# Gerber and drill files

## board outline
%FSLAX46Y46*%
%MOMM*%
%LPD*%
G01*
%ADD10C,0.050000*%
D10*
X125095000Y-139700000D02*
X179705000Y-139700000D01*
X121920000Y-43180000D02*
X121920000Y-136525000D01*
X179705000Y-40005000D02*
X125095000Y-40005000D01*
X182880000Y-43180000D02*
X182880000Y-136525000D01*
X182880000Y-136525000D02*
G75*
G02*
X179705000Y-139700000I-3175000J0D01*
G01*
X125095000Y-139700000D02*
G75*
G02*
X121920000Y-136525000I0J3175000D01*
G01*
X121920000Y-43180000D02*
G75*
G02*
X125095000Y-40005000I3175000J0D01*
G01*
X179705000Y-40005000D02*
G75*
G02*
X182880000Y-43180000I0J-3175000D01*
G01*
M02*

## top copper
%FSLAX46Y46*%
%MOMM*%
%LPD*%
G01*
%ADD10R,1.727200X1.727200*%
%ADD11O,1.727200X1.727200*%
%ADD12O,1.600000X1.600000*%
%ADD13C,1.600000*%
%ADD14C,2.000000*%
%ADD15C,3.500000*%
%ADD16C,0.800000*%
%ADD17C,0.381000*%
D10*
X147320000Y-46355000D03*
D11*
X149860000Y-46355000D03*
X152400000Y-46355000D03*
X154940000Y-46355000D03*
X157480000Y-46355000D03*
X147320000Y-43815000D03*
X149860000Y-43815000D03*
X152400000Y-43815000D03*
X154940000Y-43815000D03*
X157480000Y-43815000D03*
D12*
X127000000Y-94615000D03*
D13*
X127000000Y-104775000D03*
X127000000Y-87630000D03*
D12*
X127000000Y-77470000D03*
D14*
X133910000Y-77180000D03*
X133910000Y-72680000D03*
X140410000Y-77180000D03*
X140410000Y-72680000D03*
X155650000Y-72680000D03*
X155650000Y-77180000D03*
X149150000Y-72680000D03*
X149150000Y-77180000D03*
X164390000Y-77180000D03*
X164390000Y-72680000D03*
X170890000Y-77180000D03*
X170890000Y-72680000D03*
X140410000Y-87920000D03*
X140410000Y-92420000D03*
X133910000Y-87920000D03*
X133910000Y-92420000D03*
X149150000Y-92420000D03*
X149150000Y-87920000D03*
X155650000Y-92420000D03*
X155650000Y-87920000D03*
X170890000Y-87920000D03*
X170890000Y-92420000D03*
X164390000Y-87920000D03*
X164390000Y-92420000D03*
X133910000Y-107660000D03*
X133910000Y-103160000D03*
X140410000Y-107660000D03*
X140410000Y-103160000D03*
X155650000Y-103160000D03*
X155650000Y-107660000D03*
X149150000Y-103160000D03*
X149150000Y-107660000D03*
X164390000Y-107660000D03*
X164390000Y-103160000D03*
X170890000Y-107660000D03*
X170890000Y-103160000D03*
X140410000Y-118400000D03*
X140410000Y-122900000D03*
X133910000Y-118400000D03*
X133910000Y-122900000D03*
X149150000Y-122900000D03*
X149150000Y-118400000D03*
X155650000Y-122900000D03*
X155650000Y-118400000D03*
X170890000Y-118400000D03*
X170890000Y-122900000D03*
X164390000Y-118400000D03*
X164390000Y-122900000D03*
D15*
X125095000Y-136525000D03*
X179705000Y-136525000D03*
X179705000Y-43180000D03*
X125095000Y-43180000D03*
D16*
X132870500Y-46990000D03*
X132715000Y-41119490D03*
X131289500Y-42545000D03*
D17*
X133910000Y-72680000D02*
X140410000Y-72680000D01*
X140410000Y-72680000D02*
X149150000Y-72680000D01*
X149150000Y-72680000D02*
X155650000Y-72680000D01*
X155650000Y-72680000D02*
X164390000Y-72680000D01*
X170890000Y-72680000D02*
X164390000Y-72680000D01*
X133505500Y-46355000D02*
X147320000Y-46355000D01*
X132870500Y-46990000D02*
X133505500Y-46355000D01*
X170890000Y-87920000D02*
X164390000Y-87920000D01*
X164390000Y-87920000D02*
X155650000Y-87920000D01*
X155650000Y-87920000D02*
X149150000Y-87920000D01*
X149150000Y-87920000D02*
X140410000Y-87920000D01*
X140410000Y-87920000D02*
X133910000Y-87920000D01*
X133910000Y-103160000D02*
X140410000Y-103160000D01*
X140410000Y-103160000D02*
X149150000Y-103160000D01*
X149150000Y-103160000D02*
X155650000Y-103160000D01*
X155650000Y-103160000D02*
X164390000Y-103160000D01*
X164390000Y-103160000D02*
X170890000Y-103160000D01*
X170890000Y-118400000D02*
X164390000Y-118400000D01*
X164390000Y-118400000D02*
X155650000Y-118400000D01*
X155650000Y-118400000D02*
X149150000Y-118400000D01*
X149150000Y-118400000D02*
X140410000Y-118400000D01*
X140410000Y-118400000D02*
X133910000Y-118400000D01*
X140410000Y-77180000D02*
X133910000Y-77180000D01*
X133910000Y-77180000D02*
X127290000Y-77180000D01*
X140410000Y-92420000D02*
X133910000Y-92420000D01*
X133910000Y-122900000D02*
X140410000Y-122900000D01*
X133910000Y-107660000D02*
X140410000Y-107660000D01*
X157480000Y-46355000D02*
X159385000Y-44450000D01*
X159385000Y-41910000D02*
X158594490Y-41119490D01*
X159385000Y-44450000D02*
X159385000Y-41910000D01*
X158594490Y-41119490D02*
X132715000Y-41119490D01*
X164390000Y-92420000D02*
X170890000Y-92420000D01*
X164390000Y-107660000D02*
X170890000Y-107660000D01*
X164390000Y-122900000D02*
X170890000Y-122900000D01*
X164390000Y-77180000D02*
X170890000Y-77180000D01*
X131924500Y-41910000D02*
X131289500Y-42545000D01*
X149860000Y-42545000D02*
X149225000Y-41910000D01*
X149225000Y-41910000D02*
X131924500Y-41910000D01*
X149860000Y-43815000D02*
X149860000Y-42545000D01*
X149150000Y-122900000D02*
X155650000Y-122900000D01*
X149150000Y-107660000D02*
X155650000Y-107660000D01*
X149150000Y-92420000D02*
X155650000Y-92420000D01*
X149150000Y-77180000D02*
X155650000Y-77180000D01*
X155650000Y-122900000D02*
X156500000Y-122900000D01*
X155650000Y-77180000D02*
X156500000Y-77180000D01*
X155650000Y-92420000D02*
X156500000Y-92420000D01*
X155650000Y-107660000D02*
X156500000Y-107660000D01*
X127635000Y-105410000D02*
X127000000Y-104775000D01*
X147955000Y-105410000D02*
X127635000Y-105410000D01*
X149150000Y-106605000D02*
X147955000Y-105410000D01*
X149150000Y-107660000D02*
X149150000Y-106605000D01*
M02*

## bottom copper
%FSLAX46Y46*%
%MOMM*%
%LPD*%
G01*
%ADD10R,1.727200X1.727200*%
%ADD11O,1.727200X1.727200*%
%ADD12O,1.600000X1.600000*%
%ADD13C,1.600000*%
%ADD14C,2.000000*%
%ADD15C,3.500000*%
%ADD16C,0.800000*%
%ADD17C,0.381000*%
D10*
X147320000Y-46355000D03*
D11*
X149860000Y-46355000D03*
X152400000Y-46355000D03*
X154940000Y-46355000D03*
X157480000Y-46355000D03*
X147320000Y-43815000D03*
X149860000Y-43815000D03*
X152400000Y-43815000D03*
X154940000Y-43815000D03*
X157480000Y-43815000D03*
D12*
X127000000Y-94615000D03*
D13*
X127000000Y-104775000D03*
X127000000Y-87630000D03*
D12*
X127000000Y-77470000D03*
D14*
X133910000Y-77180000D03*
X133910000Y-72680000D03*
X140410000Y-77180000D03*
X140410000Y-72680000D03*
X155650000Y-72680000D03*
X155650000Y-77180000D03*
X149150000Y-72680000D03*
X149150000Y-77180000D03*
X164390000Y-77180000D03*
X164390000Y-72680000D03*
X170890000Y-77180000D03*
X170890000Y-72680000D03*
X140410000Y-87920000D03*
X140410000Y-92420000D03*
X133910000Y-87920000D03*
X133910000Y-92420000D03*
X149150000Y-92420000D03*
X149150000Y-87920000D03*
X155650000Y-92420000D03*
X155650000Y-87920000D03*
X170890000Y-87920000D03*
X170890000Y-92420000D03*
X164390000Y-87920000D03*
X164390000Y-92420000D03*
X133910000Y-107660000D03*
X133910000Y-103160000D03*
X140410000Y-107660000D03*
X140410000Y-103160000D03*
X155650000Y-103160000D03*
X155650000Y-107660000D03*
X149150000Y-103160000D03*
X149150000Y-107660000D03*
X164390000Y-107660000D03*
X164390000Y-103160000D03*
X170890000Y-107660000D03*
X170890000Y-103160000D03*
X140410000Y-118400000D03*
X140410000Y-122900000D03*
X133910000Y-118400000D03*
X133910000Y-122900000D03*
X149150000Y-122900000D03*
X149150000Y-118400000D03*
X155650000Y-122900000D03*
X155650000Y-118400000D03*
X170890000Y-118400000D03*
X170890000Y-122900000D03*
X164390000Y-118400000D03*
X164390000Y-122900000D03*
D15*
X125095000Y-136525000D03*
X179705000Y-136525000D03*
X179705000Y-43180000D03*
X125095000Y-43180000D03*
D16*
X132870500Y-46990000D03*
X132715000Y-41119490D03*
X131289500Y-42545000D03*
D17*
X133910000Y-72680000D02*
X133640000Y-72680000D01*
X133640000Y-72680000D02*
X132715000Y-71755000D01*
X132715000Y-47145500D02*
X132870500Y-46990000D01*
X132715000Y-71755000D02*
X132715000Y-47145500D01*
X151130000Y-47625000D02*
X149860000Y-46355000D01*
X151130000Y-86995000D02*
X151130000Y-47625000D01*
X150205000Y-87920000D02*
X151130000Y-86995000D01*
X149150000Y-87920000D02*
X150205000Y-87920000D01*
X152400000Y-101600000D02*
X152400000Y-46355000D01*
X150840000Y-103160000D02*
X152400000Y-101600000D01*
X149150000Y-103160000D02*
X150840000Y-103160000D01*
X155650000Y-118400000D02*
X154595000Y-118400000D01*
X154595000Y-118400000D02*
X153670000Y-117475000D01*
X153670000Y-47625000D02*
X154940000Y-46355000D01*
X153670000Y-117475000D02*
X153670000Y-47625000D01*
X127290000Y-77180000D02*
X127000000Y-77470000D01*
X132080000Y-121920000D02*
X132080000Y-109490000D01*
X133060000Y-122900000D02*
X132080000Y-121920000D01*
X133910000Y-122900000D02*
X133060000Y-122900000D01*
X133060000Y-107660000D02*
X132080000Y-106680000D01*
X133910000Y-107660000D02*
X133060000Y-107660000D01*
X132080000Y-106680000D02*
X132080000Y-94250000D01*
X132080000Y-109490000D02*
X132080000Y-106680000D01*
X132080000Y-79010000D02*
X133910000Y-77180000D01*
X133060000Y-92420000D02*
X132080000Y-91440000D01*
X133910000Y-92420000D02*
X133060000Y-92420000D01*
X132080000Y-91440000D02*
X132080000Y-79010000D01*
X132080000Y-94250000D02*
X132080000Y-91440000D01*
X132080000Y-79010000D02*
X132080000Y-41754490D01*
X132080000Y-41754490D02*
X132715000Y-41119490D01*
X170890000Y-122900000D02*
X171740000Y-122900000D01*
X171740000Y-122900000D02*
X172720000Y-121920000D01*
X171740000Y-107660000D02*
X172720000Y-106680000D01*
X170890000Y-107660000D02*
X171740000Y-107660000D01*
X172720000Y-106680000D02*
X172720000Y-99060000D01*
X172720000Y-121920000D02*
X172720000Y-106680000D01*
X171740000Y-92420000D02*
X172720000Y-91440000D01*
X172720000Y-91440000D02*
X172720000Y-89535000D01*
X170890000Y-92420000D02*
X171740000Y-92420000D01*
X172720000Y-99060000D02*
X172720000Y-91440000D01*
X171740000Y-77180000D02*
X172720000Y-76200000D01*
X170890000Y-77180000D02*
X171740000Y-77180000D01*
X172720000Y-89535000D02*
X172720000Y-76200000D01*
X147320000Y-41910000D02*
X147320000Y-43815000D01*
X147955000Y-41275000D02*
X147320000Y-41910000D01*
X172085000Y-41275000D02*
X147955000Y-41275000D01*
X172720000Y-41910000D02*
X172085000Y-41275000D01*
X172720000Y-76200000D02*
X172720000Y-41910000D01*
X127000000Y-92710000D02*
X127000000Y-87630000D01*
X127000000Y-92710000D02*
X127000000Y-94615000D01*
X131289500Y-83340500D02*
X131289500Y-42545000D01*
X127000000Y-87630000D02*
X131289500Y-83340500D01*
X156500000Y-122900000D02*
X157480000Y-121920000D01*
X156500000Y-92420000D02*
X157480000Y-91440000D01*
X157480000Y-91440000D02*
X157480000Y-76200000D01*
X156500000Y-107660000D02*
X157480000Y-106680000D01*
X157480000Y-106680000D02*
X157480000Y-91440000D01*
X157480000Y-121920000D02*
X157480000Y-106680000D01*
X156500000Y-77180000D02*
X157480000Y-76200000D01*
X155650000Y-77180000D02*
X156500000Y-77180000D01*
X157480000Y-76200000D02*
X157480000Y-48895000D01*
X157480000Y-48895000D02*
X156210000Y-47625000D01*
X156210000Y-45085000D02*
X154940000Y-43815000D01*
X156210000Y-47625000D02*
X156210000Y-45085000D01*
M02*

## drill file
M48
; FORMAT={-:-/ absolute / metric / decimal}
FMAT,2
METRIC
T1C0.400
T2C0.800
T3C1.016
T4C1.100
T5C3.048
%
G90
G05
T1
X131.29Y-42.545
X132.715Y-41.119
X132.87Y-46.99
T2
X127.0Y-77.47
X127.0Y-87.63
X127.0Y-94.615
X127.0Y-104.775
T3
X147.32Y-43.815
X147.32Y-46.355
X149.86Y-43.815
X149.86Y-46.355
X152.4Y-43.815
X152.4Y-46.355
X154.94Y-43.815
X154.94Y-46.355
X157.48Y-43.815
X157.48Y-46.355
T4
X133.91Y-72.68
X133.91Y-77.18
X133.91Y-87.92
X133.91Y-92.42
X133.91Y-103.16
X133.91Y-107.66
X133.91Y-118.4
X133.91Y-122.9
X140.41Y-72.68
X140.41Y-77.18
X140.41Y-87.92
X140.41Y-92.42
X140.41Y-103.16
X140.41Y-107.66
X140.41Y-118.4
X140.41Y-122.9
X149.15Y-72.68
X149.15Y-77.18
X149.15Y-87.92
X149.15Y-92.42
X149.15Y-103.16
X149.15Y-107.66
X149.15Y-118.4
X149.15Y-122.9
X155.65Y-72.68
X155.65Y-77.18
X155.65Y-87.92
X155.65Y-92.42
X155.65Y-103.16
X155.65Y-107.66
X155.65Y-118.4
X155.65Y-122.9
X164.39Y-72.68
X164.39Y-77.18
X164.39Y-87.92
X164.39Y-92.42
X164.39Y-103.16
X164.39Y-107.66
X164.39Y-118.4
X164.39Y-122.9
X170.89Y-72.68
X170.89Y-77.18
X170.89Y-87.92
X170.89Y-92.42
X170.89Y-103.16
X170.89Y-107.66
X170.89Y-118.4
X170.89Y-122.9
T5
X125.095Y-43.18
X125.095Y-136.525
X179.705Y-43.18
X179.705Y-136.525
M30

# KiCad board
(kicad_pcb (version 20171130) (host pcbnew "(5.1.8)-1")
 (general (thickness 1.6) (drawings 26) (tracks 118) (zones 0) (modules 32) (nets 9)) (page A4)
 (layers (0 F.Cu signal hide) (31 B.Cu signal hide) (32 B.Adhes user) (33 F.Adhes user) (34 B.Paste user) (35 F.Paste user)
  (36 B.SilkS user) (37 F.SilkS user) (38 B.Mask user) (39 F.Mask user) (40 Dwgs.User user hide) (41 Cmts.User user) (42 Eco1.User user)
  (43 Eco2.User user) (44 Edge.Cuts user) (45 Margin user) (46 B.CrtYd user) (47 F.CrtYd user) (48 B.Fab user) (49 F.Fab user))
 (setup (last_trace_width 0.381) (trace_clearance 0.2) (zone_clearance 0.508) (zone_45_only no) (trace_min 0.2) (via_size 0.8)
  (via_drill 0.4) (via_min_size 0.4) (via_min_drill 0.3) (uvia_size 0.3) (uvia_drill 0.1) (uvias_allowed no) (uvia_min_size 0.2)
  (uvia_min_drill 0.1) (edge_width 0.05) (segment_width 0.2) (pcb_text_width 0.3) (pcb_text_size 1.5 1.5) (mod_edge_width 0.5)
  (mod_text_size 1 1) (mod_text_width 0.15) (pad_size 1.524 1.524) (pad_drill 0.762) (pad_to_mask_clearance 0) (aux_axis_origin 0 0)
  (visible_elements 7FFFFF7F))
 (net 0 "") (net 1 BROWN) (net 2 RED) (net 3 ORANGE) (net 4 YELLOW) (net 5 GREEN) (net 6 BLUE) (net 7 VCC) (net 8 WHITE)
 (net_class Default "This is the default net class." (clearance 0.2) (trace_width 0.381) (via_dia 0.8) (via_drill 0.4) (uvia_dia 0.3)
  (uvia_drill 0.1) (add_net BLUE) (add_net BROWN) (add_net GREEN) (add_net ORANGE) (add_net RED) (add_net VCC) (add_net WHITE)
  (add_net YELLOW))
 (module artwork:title (layer F.Cu) (at 152.4 59.055)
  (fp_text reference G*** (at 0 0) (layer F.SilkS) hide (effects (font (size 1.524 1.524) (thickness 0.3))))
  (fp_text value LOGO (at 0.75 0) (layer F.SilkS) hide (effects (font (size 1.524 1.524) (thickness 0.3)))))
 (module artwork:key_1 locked (layer F.Cu) (at 137.16 69.85)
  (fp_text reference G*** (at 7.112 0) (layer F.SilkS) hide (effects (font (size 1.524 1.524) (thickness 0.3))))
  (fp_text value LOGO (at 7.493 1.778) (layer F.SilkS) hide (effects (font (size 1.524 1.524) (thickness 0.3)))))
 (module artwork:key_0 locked (layer F.Cu) (at 152.4 115.57)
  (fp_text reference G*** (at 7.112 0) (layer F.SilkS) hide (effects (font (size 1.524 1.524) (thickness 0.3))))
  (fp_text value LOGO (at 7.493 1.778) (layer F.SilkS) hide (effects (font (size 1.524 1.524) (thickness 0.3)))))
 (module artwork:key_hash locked (layer F.Cu) (at 167.64 115.57)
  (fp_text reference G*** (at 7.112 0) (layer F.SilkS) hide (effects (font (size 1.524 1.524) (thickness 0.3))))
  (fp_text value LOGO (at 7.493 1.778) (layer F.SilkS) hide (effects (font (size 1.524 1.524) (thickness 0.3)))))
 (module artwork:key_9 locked (layer F.Cu) (at 167.64 100.33)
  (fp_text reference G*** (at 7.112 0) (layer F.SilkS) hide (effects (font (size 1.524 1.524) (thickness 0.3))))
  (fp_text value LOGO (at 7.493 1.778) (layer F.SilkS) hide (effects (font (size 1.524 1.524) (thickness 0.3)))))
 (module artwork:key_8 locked (layer F.Cu) (at 152.4 100.33)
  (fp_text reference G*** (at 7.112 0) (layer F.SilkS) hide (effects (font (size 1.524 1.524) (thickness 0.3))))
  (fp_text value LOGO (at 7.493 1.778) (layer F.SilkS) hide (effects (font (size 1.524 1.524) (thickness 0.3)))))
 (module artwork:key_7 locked (layer F.Cu) (at 137.16 100.33)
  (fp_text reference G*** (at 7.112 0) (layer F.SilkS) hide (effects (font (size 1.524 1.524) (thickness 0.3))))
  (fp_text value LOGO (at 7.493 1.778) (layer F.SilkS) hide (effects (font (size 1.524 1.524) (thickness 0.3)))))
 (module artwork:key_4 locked (layer F.Cu) (at 137.16 85.09)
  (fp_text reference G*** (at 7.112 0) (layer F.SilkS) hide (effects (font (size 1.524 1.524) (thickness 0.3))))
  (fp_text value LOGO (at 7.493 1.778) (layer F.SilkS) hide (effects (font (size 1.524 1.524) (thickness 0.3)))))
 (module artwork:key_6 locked (layer F.Cu) (at 167.64 85.09)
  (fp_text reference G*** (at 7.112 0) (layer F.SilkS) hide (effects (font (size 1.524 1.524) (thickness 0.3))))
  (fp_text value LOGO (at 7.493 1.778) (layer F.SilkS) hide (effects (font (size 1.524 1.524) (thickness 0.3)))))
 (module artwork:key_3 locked (layer F.Cu) (at 167.64 69.85)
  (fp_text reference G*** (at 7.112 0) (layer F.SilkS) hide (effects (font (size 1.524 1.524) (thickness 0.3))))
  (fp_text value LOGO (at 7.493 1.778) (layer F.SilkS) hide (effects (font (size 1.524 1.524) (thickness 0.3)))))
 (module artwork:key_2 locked (layer F.Cu) (at 152.4 69.85)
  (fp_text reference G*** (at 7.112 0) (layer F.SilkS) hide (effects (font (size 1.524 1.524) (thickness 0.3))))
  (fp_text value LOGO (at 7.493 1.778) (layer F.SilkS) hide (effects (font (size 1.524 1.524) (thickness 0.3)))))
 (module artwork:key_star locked (layer F.Cu) (at 137.16 115.57)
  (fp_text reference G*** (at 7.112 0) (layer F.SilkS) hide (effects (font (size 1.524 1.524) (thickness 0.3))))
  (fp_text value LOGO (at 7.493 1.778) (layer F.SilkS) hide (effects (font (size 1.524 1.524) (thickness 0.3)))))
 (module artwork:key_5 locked (layer F.Cu) (at 152.4 85.09)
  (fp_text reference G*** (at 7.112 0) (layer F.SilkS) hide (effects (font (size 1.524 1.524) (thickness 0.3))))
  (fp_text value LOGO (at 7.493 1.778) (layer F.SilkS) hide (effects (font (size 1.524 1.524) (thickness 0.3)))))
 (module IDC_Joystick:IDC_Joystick (layer F.Cu) (at 147.32 46.355 90)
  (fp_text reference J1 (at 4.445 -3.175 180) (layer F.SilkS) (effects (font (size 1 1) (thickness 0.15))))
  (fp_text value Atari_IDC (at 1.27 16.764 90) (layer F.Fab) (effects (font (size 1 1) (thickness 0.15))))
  (pad 1 thru_hole rect (at 0 0 90) (size 1.7272 1.7272) (drill 1.016) (layers *.Cu *.Mask) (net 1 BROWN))
  (pad 2 thru_hole oval (at 0 2.54 90) (size 1.7272 1.7272) (drill 1.016) (layers *.Cu *.Mask) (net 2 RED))
  (pad 3 thru_hole oval (at 0 5.08 90) (size 1.7272 1.7272) (drill 1.016) (layers *.Cu *.Mask) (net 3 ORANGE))
  (pad 4 thru_hole oval (at 0 7.62 90) (size 1.7272 1.7272) (drill 1.016) (layers *.Cu *.Mask) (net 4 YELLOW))
  (pad 5 thru_hole oval (at 0 10.16 90) (size 1.7272 1.7272) (drill 1.016) (layers *.Cu *.Mask) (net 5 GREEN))
  (pad 6 thru_hole oval (at 2.54 0 90) (size 1.7272 1.7272) (drill 1.016) (layers *.Cu *.Mask) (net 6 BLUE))
  (pad 7 thru_hole oval (at 2.54 2.54 90) (size 1.7272 1.7272) (drill 1.016) (layers *.Cu *.Mask) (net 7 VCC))
  (pad 8 thru_hole oval (at 2.54 5.08 90) (size 1.7272 1.7272) (drill 1.016) (layers *.Cu *.Mask))
  (pad 9 thru_hole oval (at 2.54 7.62 90) (size 1.7272 1.7272) (drill 1.016) (layers *.Cu *.Mask) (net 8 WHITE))
  (pad 10 thru_hole oval (at 2.54 10.16 90) (size 1.7272 1.7272) (drill 1.016) (layers *.Cu *.Mask)))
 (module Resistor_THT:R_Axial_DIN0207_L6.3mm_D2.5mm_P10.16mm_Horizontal (layer F.Cu) (at 127 104.775 90)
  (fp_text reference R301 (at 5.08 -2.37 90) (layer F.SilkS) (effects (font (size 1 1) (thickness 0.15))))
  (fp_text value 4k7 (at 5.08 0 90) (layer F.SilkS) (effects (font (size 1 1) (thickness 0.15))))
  (pad 2 thru_hole oval (at 10.16 0 90) (size 1.6 1.6) (drill 0.8) (layers *.Cu *.Mask) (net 7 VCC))
  (pad 1 thru_hole circle (at 0 0 90) (size 1.6 1.6) (drill 0.8) (layers *.Cu *.Mask) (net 8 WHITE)))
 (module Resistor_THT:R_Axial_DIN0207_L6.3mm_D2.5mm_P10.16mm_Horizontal (layer F.Cu) (at 127 87.63 90)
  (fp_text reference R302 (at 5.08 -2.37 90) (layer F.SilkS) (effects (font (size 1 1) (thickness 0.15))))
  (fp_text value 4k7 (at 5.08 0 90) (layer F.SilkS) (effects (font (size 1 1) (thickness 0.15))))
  (pad 1 thru_hole circle (at 0 0 90) (size 1.6 1.6) (drill 0.8) (layers *.Cu *.Mask) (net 7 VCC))
  (pad 2 thru_hole oval (at 10.16 0 90) (size 1.6 1.6) (drill 0.8) (layers *.Cu *.Mask) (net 5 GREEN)))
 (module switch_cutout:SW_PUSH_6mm (layer F.Cu) (at 137.16 74.93)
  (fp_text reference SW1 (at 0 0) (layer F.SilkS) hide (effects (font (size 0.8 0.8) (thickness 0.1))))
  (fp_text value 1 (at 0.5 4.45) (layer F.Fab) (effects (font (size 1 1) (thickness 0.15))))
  (pad 2 thru_hole circle (at -3.25 2.25 90) (size 2 2) (drill 1.1) (layers *.Cu *.Mask) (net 5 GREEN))
  (pad 1 thru_hole circle (at -3.25 -2.25 90) (size 2 2) (drill 1.1) (layers *.Cu *.Mask) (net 1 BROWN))
  (pad 2 thru_hole circle (at 3.25 2.25 90) (size 2 2) (drill 1.1) (layers *.Cu *.Mask) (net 5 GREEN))
  (pad 1 thru_hole circle (at 3.25 -2.25 90) (size 2 2) (drill 1.1) (layers *.Cu *.Mask) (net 1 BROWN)))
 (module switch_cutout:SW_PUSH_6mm (layer F.Cu) (at 152.4 74.93)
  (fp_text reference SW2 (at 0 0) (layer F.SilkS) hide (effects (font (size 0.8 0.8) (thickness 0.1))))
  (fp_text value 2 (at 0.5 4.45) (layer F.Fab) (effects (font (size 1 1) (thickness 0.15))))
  (pad 1 thru_hole circle (at 3.25 -2.25 90) (size 2 2) (drill 1.1) (layers *.Cu *.Mask) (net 1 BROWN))
  (pad 2 thru_hole circle (at 3.25 2.25 90) (size 2 2) (drill 1.1) (layers *.Cu *.Mask) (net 8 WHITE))
  (pad 1 thru_hole circle (at -3.25 -2.25 90) (size 2 2) (drill 1.1) (layers *.Cu *.Mask) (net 1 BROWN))
  (pad 2 thru_hole circle (at -3.25 2.25 90) (size 2 2) (drill 1.1) (layers *.Cu *.Mask) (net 8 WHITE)))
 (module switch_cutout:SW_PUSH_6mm (layer F.Cu) (at 167.64 74.93)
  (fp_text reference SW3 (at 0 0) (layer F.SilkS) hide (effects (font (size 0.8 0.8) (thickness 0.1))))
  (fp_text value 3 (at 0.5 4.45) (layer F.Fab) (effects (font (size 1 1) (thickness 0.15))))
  (pad 2 thru_hole circle (at -3.25 2.25 90) (size 2 2) (drill 1.1) (layers *.Cu *.Mask) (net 6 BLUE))
  (pad 1 thru_hole circle (at -3.25 -2.25 90) (size 2 2) (drill 1.1) (layers *.Cu *.Mask) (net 1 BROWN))
  (pad 2 thru_hole circle (at 3.25 2.25 90) (size 2 2) (drill 1.1) (layers *.Cu *.Mask) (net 6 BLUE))
  (pad 1 thru_hole circle (at 3.25 -2.25 90) (size 2 2) (drill 1.1) (layers *.Cu *.Mask) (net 1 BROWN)))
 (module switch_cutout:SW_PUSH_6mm (layer F.Cu) (at 137.16 90.17)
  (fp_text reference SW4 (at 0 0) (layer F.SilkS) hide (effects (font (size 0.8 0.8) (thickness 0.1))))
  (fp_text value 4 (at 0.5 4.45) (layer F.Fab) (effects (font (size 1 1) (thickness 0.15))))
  (pad 1 thru_hole circle (at 3.25 -2.25 90) (size 2 2) (drill 1.1) (layers *.Cu *.Mask) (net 2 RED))
  (pad 2 thru_hole circle (at 3.25 2.25 90) (size 2 2) (drill 1.1) (layers *.Cu *.Mask) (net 5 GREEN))
  (pad 1 thru_hole circle (at -3.25 -2.25 90) (size 2 2) (drill 1.1) (layers *.Cu *.Mask) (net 2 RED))
  (pad 2 thru_hole circle (at -3.25 2.25 90) (size 2 2) (drill 1.1) (layers *.Cu *.Mask) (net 5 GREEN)))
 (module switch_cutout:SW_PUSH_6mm (layer F.Cu) (at 152.4 90.17)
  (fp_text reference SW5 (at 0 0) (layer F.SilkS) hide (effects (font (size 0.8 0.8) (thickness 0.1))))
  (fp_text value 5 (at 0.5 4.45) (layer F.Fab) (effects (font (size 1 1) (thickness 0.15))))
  (pad 2 thru_hole circle (at -3.25 2.25 90) (size 2 2) (drill 1.1) (layers *.Cu *.Mask) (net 8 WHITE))
  (pad 1 thru_hole circle (at -3.25 -2.25 90) (size 2 2) (drill 1.1) (layers *.Cu *.Mask) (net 2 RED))
  (pad 2 thru_hole circle (at 3.25 2.25 90) (size 2 2) (drill 1.1) (layers *.Cu *.Mask) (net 8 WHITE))
  (pad 1 thru_hole circle (at 3.25 -2.25 90) (size 2 2) (drill 1.1) (layers *.Cu *.Mask) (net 2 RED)))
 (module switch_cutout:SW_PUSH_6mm (layer F.Cu) (at 167.64 90.17)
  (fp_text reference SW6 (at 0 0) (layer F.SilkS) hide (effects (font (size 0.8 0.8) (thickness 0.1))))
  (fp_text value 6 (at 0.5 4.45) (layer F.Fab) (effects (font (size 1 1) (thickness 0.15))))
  (pad 1 thru_hole circle (at 3.25 -2.25 90) (size 2 2) (drill 1.1) (layers *.Cu *.Mask) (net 2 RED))
  (pad 2 thru_hole circle (at 3.25 2.25 90) (size 2 2) (drill 1.1) (layers *.Cu *.Mask) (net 6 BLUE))
  (pad 1 thru_hole circle (at -3.25 -2.25 90) (size 2 2) (drill 1.1) (layers *.Cu *.Mask) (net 2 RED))
  (pad 2 thru_hole circle (at -3.25 2.25 90) (size 2 2) (drill 1.1) (layers *.Cu *.Mask) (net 6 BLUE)))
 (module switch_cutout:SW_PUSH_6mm (layer F.Cu) (at 137.16 105.41)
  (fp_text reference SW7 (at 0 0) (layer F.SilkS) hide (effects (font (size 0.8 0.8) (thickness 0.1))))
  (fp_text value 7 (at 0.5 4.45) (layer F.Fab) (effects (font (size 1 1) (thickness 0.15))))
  (pad 2 thru_hole circle (at -3.25 2.25 90) (size 2 2) (drill 1.1) (layers *.Cu *.Mask) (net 5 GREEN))
  (pad 1 thru_hole circle (at -3.25 -2.25 90) (size 2 2) (drill 1.1) (layers *.Cu *.Mask) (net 3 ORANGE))
  (pad 2 thru_hole circle (at 3.25 2.25 90) (size 2 2) (drill 1.1) (layers *.Cu *.Mask) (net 5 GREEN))
  (pad 1 thru_hole circle (at 3.25 -2.25 90) (size 2 2) (drill 1.1) (layers *.Cu *.Mask) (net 3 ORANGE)))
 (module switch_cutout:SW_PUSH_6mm (layer F.Cu) (at 152.4 105.41)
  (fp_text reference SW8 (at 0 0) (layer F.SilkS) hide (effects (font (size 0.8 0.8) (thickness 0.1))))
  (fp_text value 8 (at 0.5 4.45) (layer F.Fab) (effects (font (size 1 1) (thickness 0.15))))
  (pad 1 thru_hole circle (at 3.25 -2.25 90) (size 2 2) (drill 1.1) (layers *.Cu *.Mask) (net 3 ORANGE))
  (pad 2 thru_hole circle (at 3.25 2.25 90) (size 2 2) (drill 1.1) (layers *.Cu *.Mask) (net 8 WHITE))
  (pad 1 thru_hole circle (at -3.25 -2.25 90) (size 2 2) (drill 1.1) (layers *.Cu *.Mask) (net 3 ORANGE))
  (pad 2 thru_hole circle (at -3.25 2.25 90) (size 2 2) (drill 1.1) (layers *.Cu *.Mask) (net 8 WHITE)))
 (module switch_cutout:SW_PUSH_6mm (layer F.Cu) (at 167.64 105.41)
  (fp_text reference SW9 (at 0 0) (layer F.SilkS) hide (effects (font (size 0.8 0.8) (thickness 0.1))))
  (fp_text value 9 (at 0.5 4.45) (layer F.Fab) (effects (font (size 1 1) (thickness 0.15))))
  (pad 2 thru_hole circle (at -3.25 2.25 90) (size 2 2) (drill 1.1) (layers *.Cu *.Mask) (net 6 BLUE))
  (pad 1 thru_hole circle (at -3.25 -2.25 90) (size 2 2) (drill 1.1) (layers *.Cu *.Mask) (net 3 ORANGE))
  (pad 2 thru_hole circle (at 3.25 2.25 90) (size 2 2) (drill 1.1) (layers *.Cu *.Mask) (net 6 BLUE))
  (pad 1 thru_hole circle (at 3.25 -2.25 90) (size 2 2) (drill 1.1) (layers *.Cu *.Mask) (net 3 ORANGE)))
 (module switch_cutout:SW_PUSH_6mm (layer F.Cu) (at 137.16 120.65)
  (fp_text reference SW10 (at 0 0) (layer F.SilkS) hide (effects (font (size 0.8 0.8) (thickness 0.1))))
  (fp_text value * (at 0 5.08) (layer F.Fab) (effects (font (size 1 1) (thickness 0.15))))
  (pad 1 thru_hole circle (at 3.25 -2.25 90) (size 2 2) (drill 1.1) (layers *.Cu *.Mask) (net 4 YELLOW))
  (pad 2 thru_hole circle (at 3.25 2.25 90) (size 2 2) (drill 1.1) (layers *.Cu *.Mask) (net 5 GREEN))
  (pad 1 thru_hole circle (at -3.25 -2.25 90) (size 2 2) (drill 1.1) (layers *.Cu *.Mask) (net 4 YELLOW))
  (pad 2 thru_hole circle (at -3.25 2.25 90) (size 2 2) (drill 1.1) (layers *.Cu *.Mask) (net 5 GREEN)))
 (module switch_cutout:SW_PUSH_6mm (layer F.Cu) (at 152.4 120.65)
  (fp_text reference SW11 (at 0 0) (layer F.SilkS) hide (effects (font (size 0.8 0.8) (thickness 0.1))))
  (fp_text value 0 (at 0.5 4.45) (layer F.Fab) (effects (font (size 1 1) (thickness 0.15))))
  (pad 2 thru_hole circle (at -3.25 2.25 90) (size 2 2) (drill 1.1) (layers *.Cu *.Mask) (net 8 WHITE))
  (pad 1 thru_hole circle (at -3.25 -2.25 90) (size 2 2) (drill 1.1) (layers *.Cu *.Mask) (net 4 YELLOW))
  (pad 2 thru_hole circle (at 3.25 2.25 90) (size 2 2) (drill 1.1) (layers *.Cu *.Mask) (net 8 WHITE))
  (pad 1 thru_hole circle (at 3.25 -2.25 90) (size 2 2) (drill 1.1) (layers *.Cu *.Mask) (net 4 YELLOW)))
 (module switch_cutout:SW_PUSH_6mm (layer F.Cu) (at 167.64 120.65)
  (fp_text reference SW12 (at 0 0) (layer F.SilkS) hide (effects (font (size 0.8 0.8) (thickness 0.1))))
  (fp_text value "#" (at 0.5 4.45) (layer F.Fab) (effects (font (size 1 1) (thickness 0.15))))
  (pad 1 thru_hole circle (at 3.25 -2.25 90) (size 2 2) (drill 1.1) (layers *.Cu *.Mask) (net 4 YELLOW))
  (pad 2 thru_hole circle (at 3.25 2.25 90) (size 2 2) (drill 1.1) (layers *.Cu *.Mask) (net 6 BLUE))
  (pad 1 thru_hole circle (at -3.25 -2.25 90) (size 2 2) (drill 1.1) (layers *.Cu *.Mask) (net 4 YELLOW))
  (pad 2 thru_hole circle (at -3.25 2.25 90) (size 2 2) (drill 1.1) (layers *.Cu *.Mask) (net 6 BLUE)))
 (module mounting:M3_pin (layer F.Cu) (at 125.095 136.525)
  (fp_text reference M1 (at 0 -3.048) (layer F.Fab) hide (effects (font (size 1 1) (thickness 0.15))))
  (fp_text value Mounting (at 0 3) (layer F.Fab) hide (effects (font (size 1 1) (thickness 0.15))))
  (pad 1 thru_hole circle (at 0 0) (size 3.5 3.5) (drill 3.048) (layers *.Cu *.Mask) (solder_mask_margin 0.8)))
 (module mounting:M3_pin (layer F.Cu) (at 179.705 136.525)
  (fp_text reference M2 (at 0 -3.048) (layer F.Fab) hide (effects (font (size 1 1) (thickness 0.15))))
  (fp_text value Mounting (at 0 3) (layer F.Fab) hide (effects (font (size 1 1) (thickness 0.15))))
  (pad 1 thru_hole circle (at 0 0) (size 3.5 3.5) (drill 3.048) (layers *.Cu *.Mask) (solder_mask_margin 0.8)))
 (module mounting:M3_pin (layer F.Cu) (at 179.705 43.18)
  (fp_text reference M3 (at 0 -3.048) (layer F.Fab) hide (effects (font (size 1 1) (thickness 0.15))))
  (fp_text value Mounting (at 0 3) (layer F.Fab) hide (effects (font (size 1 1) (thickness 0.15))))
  (pad 1 thru_hole circle (at 0 0) (size 3.5 3.5) (drill 3.048) (layers *.Cu *.Mask) (solder_mask_margin 0.8)))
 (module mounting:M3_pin (layer F.Cu) (at 125.095 43.18)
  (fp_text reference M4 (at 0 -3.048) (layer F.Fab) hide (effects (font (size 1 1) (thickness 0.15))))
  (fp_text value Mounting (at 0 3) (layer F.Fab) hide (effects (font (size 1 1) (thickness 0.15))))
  (pad 1 thru_hole circle (at 0 0) (size 3.5 3.5) (drill 3.048) (layers *.Cu *.Mask) (solder_mask_margin 0.8)))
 (gr_line (start 125.095 139.7) (end 179.705 139.7) (layer Edge.Cuts) (width 0.05))
 (gr_line (start 121.92 43.18) (end 121.92 136.525) (layer Edge.Cuts) (width 0.05))
 (gr_line (start 179.705 40.005) (end 125.095 40.005) (layer Edge.Cuts) (width 0.05))
 (gr_line (start 182.88 43.18) (end 182.88 136.525) (layer Edge.Cuts) (width 0.05))
 (gr_arc (start 179.705 136.525) (end 179.705 139.7) (angle -90) (layer Edge.Cuts) (width 0.05))
 (gr_arc (start 125.095 136.525) (end 121.92 136.525) (angle -90) (layer Edge.Cuts) (width 0.05))
 (gr_arc (start 125.095 43.18) (end 125.095 40.005) (angle -90) (layer Edge.Cuts) (width 0.05))
 (gr_arc (start 179.705 43.18) (end 182.88 43.18) (angle -90) (layer Edge.Cuts) (width 0.05))
 (segment (start 133.91 72.68) (end 140.41 72.68) (width 0.381) (layer F.Cu) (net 1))
 (segment (start 140.41 72.68) (end 149.15 72.68) (width 0.381) (layer F.Cu) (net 1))
 (segment (start 149.15 72.68) (end 155.65 72.68) (width 0.381) (layer F.Cu) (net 1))
 (segment (start 155.65 72.68) (end 164.39 72.68) (width 0.381) (layer F.Cu) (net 1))
 (segment (start 170.89 72.68) (end 164.39 72.68) (width 0.381) (layer F.Cu) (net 1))
 (segment (start 133.91 72.68) (end 133.64 72.68) (width 0.381) (layer B.Cu) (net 1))
 (segment (start 133.64 72.68) (end 132.715 71.755) (width 0.381) (layer B.Cu) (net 1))
 (via (at 132.8705 46.99) (size 0.8) (drill 0.4) (layers F.Cu B.Cu) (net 1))
 (segment (start 132.715 47.1455) (end 132.8705 46.99) (width 0.381) (layer B.Cu) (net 1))
 (segment (start 132.715 71.755) (end 132.715 47.1455) (width 0.381) (layer B.Cu) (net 1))
 (segment (start 133.5055 46.355) (end 147.32 46.355) (width 0.381) (layer F.Cu) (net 1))
 (segment (start 132.8705 46.99) (end 133.5055 46.355) (width 0.381) (layer F.Cu) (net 1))
 (segment (start 170.89 87.92) (end 164.39 87.92) (width 0.381) (layer F.Cu) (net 2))
 (segment (start 164.39 87.92) (end 155.65 87.92) (width 0.381) (layer F.Cu) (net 2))
 (segment (start 155.65 87.92) (end 149.15 87.92) (width 0.381) (layer F.Cu) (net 2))
 (segment (start 149.15 87.92) (end 140.41 87.92) (width 0.381) (layer F.Cu) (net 2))
 (segment (start 140.41 87.92) (end 133.91 87.92) (width 0.381) (layer F.Cu) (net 2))
 (segment (start 151.13 47.625) (end 149.86 46.355) (width 0.381) (layer B.Cu) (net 2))
 (segment (start 151.13 86.995) (end 151.13 47.625) (width 0.381) (layer B.Cu) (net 2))
 (segment (start 150.205 87.92) (end 151.13 86.995) (width 0.381) (layer B.Cu) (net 2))
 (segment (start 149.15 87.92) (end 150.205 87.92) (width 0.381) (layer B.Cu) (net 2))
 (segment (start 133.91 103.16) (end 140.41 103.16) (width 0.381) (layer F.Cu) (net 3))
 (segment (start 140.41 103.16) (end 149.15 103.16) (width 0.381) (layer F.Cu) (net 3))
 (segment (start 149.15 103.16) (end 155.65 103.16) (width 0.381) (layer F.Cu) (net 3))
 (segment (start 155.65 103.16) (end 164.39 103.16) (width 0.381) (layer F.Cu) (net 3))
 (segment (start 164.39 103.16) (end 170.89 103.16) (width 0.381) (layer F.Cu) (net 3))
 (segment (start 152.4 101.6) (end 152.4 46.355) (width 0.381) (layer B.Cu) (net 3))
 (segment (start 150.84 103.16) (end 152.4 101.6) (width 0.381) (layer B.Cu) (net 3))
 (segment (start 149.15 103.16) (end 150.84 103.16) (width 0.381) (layer B.Cu) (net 3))
 (segment (start 170.89 118.4) (end 164.39 118.4) (width 0.381) (layer F.Cu) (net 4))
 (segment (start 164.39 118.4) (end 155.65 118.4) (width 0.381) (layer F.Cu) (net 4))
 (segment (start 155.65 118.4) (end 149.15 118.4) (width 0.381) (layer F.Cu) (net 4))
 (segment (start 149.15 118.4) (end 140.41 118.4) (width 0.381) (layer F.Cu) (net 4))
 (segment (start 140.41 118.4) (end 133.91 118.4) (width 0.381) (layer F.Cu) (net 4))
 (segment (start 155.65 118.4) (end 154.595 118.4) (width 0.381) (layer B.Cu) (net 4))
 (segment (start 154.595 118.4) (end 153.67 117.475) (width 0.381) (layer B.Cu) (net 4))
 (segment (start 153.67 47.625) (end 154.94 46.355) (width 0.381) (layer B.Cu) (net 4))
 (segment (start 153.67 117.475) (end 153.67 47.625) (width 0.381) (layer B.Cu) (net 4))
 (segment (start 140.41 77.18) (end 133.91 77.18) (width 0.381) (layer F.Cu) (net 5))
 (segment (start 127.29 77.18) (end 127 77.47) (width 0.381) (layer B.Cu) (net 5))
 (segment (start 133.91 77.18) (end 127.29 77.18) (width 0.381) (layer F.Cu) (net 5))
 (segment (start 140.41 92.42) (end 133.91 92.42) (width 0.381) (layer F.Cu) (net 5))
 (segment (start 133.91 122.9) (end 140.41 122.9) (width 0.381) (layer F.Cu) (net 5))
 (segment (start 133.91 107.66) (end 140.41 107.66) (width 0.381) (layer F.Cu) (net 5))
 (segment (start 132.08 121.92) (end 132.08 109.49) (width 0.381) (layer B.Cu) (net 5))
 (segment (start 133.06 122.9) (end 132.08 121.92) (width 0.381) (layer B.Cu) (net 5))
 (segment (start 133.91 122.9) (end 133.06 122.9) (width 0.381) (layer B.Cu) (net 5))
 (segment (start 133.06 107.66) (end 132.08 106.68) (width 0.381) (layer B.Cu) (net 5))
 (segment (start 133.91 107.66) (end 133.06 107.66) (width 0.381) (layer B.Cu) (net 5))
 (segment (start 132.08 106.68) (end 132.08 94.25) (width 0.381) (layer B.Cu) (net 5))
 (segment (start 132.08 109.49) (end 132.08 106.68) (width 0.381) (layer B.Cu) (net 5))
 (segment (start 132.08 79.01) (end 133.91 77.18) (width 0.381) (layer B.Cu) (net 5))
 (segment (start 133.06 92.42) (end 132.08 91.44) (width 0.381) (layer B.Cu) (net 5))
 (segment (start 133.91 92.42) (end 133.06 92.42) (width 0.381) (layer B.Cu) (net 5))
 (segment (start 132.08 91.44) (end 132.08 79.01) (width 0.381) (layer B.Cu) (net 5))
 (segment (start 132.08 94.25) (end 132.08 91.44) (width 0.381) (layer B.Cu) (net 5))
 (segment (start 157.48 46.355) (end 159.385 44.45) (width 0.381) (layer F.Cu) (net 5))
 (via (at 132.715 41.11949) (size 0.8) (drill 0.4) (layers F.Cu B.Cu) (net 5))
 (segment (start 159.385 41.91) (end 158.59449 41.11949) (width 0.381) (layer F.Cu) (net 5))
 (segment (start 132.08 79.01) (end 132.08 41.75449) (width 0.381) (layer B.Cu) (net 5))
 (segment (start 132.08 41.75449) (end 132.715 41.11949) (width 0.381) (layer B.Cu) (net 5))
 (segment (start 159.385 44.45) (end 159.385 41.91) (width 0.381) (layer F.Cu) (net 5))
 (segment (start 158.59449 41.11949) (end 132.715 41.11949) (width 0.381) (layer F.Cu) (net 5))
 (segment (start 164.39 92.42) (end 170.89 92.42) (width 0.381) (layer F.Cu) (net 6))
 (segment (start 164.39 107.66) (end 170.89 107.66) (width 0.381) (layer F.Cu) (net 6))
 (segment (start 164.39 122.9) (end 170.89 122.9) (width 0.381) (layer F.Cu) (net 6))
 (segment (start 164.39 77.18) (end 170.89 77.18) (width 0.381) (layer F.Cu) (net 6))
 (segment (start 170.89 122.9) (end 171.74 122.9) (width 0.381) (layer B.Cu) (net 6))
 (segment (start 171.74 122.9) (end 172.72 121.92) (width 0.381) (layer B.Cu) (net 6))
 (segment (start 171.74 107.66) (end 172.72 106.68) (width 0.381) (layer B.Cu) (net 6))
 (segment (start 170.89 107.66) (end 171.74 107.66) (width 0.381) (layer B.Cu) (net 6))
 (segment (start 172.72 106.68) (end 172.72 99.06) (width 0.381) (layer B.Cu) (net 6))
 (segment (start 172.72 121.92) (end 172.72 106.68) (width 0.381) (layer B.Cu) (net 6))
 (segment (start 171.74 92.42) (end 172.72 91.44) (width 0.381) (layer B.Cu) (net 6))
 (segment (start 172.72 91.44) (end 172.72 89.535) (width 0.381) (layer B.Cu) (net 6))
 (segment (start 170.89 92.42) (end 171.74 92.42) (width 0.381) (layer B.Cu) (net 6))
 (segment (start 172.72 99.06) (end 172.72 91.44) (width 0.381) (layer B.Cu) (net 6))
 (segment (start 171.74 77.18) (end 172.72 76.2) (width 0.381) (layer B.Cu) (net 6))
 (segment (start 170.89 77.18) (end 171.74 77.18) (width 0.381) (layer B.Cu) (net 6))
 (segment (start 172.72 89.535) (end 172.72 76.2) (width 0.381) (layer B.Cu) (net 6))
 (segment (start 147.32 41.91) (end 147.32 43.815) (width 0.381) (layer B.Cu) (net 6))
 (segment (start 147.955 41.275) (end 147.32 41.91) (width 0.381) (layer B.Cu) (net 6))
 (segment (start 172.085 41.275) (end 147.955 41.275) (width 0.381) (layer B.Cu) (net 6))
 (segment (start 172.72 41.91) (end 172.085 41.275) (width 0.381) (layer B.Cu) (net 6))
 (segment (start 172.72 76.2) (end 172.72 41.91) (width 0.381) (layer B.Cu) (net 6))
 (segment (start 127 92.71) (end 127 87.63) (width 0.381) (layer B.Cu) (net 7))
 (segment (start 127 92.71) (end 127 94.615) (width 0.381) (layer B.Cu) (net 7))
 (via (at 131.2895 42.545) (size 0.8) (drill 0.4) (layers F.Cu B.Cu) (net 7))
 (segment (start 131.2895 83.3405) (end 131.2895 42.545) (width 0.381) (layer B.Cu) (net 7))
 (segment (start 127 87.63) (end 131.2895 83.3405) (width 0.381) (layer B.Cu) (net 7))
 (segment (start 131.9245 41.91) (end 131.2895 42.545) (width 0.381) (layer F.Cu) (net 7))
 (segment (start 149.86 42.545) (end 149.225 41.91) (width 0.381) (layer F.Cu) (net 7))
 (segment (start 149.225 41.91) (end 131.9245 41.91) (width 0.381) (layer F.Cu) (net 7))
 (segment (start 149.86 43.815) (end 149.86 42.545) (width 0.381) (layer F.Cu) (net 7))
 (segment (start 149.15 122.9) (end 155.65 122.9) (width 0.381) (layer F.Cu) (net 8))
 (segment (start 149.15 107.66) (end 155.65 107.66) (width 0.381) (layer F.Cu) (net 8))
 (segment (start 149.15 92.42) (end 155.65 92.42) (width 0.381) (layer F.Cu) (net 8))
 (segment (start 149.15 77.18) (end 155.65 77.18) (width 0.381) (layer F.Cu) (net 8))
 (segment (start 156.5 122.9) (end 157.48 121.92) (width 0.381) (layer B.Cu) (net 8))
 (segment (start 155.65 122.9) (end 156.5 122.9) (width 0.381) (layer F.Cu) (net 8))
 (segment (start 155.65 77.18) (end 156.5 77.18) (width 0.381) (layer F.Cu) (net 8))
 (segment (start 156.5 92.42) (end 157.48 91.44) (width 0.381) (layer B.Cu) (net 8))
 (segment (start 155.65 92.42) (end 156.5 92.42) (width 0.381) (layer F.Cu) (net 8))
 (segment (start 157.48 91.44) (end 157.48 76.2) (width 0.381) (layer B.Cu) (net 8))
 (segment (start 156.5 107.66) (end 157.48 106.68) (width 0.381) (layer B.Cu) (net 8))
 (segment (start 155.65 107.66) (end 156.5 107.66) (width 0.381) (layer F.Cu) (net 8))
 (segment (start 157.48 106.68) (end 157.48 91.44) (width 0.381) (layer B.Cu) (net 8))
 (segment (start 157.48 121.92) (end 157.48 106.68) (width 0.381) (layer B.Cu) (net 8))
 (segment (start 127.635 105.41) (end 127 104.775) (width 0.381) (layer F.Cu) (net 8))
 (segment (start 147.955 105.41) (end 127.635 105.41) (width 0.381) (layer F.Cu) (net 8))
 (segment (start 149.15 106.605) (end 147.955 105.41) (width 0.381) (layer F.Cu) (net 8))
 (segment (start 149.15 107.66) (end 149.15 106.605) (width 0.381) (layer F.Cu) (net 8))
 (segment (start 156.5 77.18) (end 157.48 76.2) (width 0.381) (layer B.Cu) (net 8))
 (segment (start 155.65 77.18) (end 156.5 77.18) (width 0.381) (layer B.Cu) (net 8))
 (segment (start 157.48 76.2) (end 157.48 48.895) (width 0.381) (layer B.Cu) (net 8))
 (segment (start 157.48 48.895) (end 156.21 47.625) (width 0.381) (layer B.Cu) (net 8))
 (segment (start 156.21 45.085) (end 154.94 43.815) (width 0.381) (layer B.Cu) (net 8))
 (segment (start 156.21 47.625) (end 156.21 45.085) (width 0.381) (layer B.Cu) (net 8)))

